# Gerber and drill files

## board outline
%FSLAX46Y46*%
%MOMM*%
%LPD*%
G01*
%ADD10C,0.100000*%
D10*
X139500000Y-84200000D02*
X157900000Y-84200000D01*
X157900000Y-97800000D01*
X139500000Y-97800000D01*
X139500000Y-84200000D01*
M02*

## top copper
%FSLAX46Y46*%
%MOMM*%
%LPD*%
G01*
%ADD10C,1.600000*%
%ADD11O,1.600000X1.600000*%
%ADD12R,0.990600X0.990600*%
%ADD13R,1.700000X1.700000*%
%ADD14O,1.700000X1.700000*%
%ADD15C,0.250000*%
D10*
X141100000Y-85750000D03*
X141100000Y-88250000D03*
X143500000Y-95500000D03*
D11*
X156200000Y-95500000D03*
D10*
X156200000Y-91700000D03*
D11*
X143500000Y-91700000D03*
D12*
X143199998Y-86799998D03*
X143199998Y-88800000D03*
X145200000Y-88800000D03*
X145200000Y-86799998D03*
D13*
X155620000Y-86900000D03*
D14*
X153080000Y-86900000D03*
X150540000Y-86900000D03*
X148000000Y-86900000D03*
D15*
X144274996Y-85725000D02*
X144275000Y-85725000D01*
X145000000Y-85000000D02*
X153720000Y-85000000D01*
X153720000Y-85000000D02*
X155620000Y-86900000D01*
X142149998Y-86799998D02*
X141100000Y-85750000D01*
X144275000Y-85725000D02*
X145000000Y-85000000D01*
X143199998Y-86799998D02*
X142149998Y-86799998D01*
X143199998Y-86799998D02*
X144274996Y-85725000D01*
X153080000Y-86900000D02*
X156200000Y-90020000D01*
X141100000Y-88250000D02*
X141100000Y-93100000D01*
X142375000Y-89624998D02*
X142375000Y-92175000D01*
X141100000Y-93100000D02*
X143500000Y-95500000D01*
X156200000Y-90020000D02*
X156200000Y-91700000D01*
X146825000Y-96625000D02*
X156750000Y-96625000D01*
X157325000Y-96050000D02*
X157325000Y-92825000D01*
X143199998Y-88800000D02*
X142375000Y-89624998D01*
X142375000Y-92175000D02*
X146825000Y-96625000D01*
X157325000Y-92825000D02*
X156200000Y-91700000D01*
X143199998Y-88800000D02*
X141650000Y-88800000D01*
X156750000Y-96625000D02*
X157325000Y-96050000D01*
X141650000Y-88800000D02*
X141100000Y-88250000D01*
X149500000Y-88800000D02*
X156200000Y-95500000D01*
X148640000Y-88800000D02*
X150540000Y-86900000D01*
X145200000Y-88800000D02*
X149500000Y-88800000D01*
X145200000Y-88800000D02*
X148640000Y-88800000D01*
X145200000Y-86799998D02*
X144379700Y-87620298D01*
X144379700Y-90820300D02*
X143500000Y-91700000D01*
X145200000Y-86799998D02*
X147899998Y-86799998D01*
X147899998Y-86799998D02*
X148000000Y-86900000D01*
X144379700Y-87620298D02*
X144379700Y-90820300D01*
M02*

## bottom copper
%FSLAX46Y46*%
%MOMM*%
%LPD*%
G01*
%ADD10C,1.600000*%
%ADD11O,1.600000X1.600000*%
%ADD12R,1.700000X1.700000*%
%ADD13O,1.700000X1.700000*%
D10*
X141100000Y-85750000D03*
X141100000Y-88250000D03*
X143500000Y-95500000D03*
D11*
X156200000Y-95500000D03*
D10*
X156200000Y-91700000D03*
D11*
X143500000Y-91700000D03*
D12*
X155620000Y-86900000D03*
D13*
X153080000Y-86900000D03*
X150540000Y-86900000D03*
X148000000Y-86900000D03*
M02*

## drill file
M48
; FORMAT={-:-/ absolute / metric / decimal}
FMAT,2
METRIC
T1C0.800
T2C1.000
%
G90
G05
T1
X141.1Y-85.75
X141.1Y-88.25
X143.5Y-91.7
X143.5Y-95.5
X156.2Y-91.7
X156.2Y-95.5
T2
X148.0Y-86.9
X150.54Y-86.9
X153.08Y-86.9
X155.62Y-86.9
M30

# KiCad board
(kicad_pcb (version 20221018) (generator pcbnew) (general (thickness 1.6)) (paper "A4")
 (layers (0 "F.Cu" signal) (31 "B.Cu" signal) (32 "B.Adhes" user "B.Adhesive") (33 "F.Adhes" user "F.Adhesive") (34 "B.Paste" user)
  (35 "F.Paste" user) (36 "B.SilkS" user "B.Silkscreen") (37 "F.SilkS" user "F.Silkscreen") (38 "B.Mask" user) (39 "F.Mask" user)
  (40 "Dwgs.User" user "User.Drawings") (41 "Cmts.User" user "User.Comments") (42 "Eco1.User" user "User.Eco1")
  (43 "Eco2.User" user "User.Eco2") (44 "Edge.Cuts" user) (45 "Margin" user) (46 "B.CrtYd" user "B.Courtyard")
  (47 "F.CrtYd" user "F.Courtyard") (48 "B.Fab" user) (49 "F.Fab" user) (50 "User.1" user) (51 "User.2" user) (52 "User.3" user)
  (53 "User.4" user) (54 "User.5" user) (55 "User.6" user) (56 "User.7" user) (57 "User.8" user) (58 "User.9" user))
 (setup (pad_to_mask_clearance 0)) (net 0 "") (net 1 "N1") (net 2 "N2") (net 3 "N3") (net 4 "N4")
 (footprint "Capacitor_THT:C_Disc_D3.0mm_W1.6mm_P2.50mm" (layer "F.Cu") (at 141.1 85.75 -90)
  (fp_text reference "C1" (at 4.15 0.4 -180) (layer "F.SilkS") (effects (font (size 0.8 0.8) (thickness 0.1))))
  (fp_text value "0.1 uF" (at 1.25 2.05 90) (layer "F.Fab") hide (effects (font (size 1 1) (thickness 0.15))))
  (pad "1" thru_hole circle (at 0 0 270) (size 1.6 1.6) (drill 0.8) (layers "*.Cu" "*.Mask") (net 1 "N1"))
  (pad "2" thru_hole circle (at 2.5 0 270) (size 1.6 1.6) (drill 0.8) (layers "*.Cu" "*.Mask") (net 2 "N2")))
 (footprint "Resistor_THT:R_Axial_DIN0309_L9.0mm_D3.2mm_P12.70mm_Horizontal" (layer "F.Cu") (at 143.5 95.5)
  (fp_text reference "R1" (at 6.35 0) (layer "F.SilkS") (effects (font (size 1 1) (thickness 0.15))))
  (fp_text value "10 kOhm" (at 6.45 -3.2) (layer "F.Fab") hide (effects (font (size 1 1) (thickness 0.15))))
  (pad "1" thru_hole circle (at 0 0) (size 1.6 1.6) (drill 0.8) (layers "*.Cu" "*.Mask") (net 2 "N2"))
  (pad "2" thru_hole oval (at 12.7 0) (size 1.6 1.6) (drill 0.8) (layers "*.Cu" "*.Mask") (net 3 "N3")))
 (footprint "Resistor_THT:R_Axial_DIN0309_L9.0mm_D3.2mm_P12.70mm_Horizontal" (layer "F.Cu") (at 156.2 91.7 180)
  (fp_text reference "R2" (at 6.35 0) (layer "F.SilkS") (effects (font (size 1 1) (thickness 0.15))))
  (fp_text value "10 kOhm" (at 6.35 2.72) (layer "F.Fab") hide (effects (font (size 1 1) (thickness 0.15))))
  (pad "1" thru_hole circle (at 0 0 180) (size 1.6 1.6) (drill 0.8) (layers "*.Cu" "*.Mask") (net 2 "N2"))
  (pad "2" thru_hole oval (at 12.7 0 180) (size 1.6 1.6) (drill 0.8) (layers "*.Cu" "*.Mask") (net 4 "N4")))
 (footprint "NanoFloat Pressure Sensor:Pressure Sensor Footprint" (layer "F.Cu") (at 144.199999 87.799999)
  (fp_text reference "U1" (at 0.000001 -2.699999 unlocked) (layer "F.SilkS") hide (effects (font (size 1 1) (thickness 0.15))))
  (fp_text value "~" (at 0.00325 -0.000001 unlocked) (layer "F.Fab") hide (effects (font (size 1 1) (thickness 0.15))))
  (pad "1" smd rect (at -1.000001 -1.000001) (size 0.9906 0.9906) (layers "F.Cu" "F.Paste" "F.Mask") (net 1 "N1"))
  (pad "2" smd rect (at -1.000001 1.000001) (size 0.9906 0.9906) (layers "F.Cu" "F.Paste" "F.Mask") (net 2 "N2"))
  (pad "3" smd rect (at 1.000001 1.000001) (size 0.9906 0.9906) (layers "F.Cu" "F.Paste" "F.Mask") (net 3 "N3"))
  (pad "4" smd rect (at 1.000001 -1.000001) (size 0.9906 0.9906) (layers "F.Cu" "F.Paste" "F.Mask") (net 4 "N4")))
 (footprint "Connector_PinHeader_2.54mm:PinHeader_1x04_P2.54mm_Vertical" (layer "B.Cu") (at 155.62 86.9 90)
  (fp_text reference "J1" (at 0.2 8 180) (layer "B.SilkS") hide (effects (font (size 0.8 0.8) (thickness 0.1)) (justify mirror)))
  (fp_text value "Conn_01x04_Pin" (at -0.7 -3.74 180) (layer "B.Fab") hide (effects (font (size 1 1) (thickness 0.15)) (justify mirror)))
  (pad "1" thru_hole rect (at 0 0 90) (size 1.7 1.7) (drill 1) (layers "*.Cu" "*.Mask") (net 1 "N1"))
  (pad "2" thru_hole oval (at 0 -2.54 90) (size 1.7 1.7) (drill 1) (layers "*.Cu" "*.Mask") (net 2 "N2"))
  (pad "3" thru_hole oval (at 0 -5.08 90) (size 1.7 1.7) (drill 1) (layers "*.Cu" "*.Mask") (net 3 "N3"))
  (pad "4" thru_hole oval (at 0 -7.62 90) (size 1.7 1.7) (drill 1) (layers "*.Cu" "*.Mask") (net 4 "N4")))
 (gr_rect (start 139.5 84.2) (end 157.9 97.8) (stroke (width 0.1) (type default)) (fill none) (layer "Edge.Cuts"))
 (segment (start 144.274996 85.725) (end 144.275 85.725) (width 0.25) (layer "F.Cu") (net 1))
 (segment (start 145 85) (end 153.72 85) (width 0.25) (layer "F.Cu") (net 1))
 (segment (start 153.72 85) (end 155.62 86.9) (width 0.25) (layer "F.Cu") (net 1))
 (segment (start 142.149998 86.799998) (end 141.1 85.75) (width 0.25) (layer "F.Cu") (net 1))
 (segment (start 144.275 85.725) (end 145 85) (width 0.25) (layer "F.Cu") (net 1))
 (segment (start 143.199998 86.799998) (end 142.149998 86.799998) (width 0.25) (layer "F.Cu") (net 1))
 (segment (start 143.199998 86.799998) (end 144.274996 85.725) (width 0.25) (layer "F.Cu") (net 1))
 (segment (start 153.08 86.9) (end 156.2 90.02) (width 0.25) (layer "F.Cu") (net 2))
 (segment (start 141.1 88.25) (end 141.1 93.1) (width 0.25) (layer "F.Cu") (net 2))
 (segment (start 142.375 89.624998) (end 142.375 92.175) (width 0.25) (layer "F.Cu") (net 2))
 (segment (start 141.1 93.1) (end 143.5 95.5) (width 0.25) (layer "F.Cu") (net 2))
 (segment (start 156.2 90.02) (end 156.2 91.7) (width 0.25) (layer "F.Cu") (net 2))
 (segment (start 146.825 96.625) (end 156.75 96.625) (width 0.25) (layer "F.Cu") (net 2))
 (segment (start 157.325 96.05) (end 157.325 92.825) (width 0.25) (layer "F.Cu") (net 2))
 (segment (start 143.199998 88.8) (end 142.375 89.624998) (width 0.25) (layer "F.Cu") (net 2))
 (segment (start 142.375 92.175) (end 146.825 96.625) (width 0.25) (layer "F.Cu") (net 2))
 (segment (start 157.325 92.825) (end 156.2 91.7) (width 0.25) (layer "F.Cu") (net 2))
 (segment (start 143.199998 88.8) (end 141.65 88.8) (width 0.25) (layer "F.Cu") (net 2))
 (segment (start 156.75 96.625) (end 157.325 96.05) (width 0.25) (layer "F.Cu") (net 2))
 (segment (start 141.65 88.8) (end 141.1 88.25) (width 0.25) (layer "F.Cu") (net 2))
 (segment (start 149.5 88.8) (end 156.2 95.5) (width 0.25) (layer "F.Cu") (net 3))
 (segment (start 148.64 88.8) (end 150.54 86.9) (width 0.25) (layer "F.Cu") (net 3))
 (segment (start 145.2 88.8) (end 149.5 88.8) (width 0.25) (layer "F.Cu") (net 3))
 (segment (start 145.2 88.8) (end 148.64 88.8) (width 0.25) (layer "F.Cu") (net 3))
 (segment (start 145.2 86.799998) (end 144.3797 87.620298) (width 0.25) (layer "F.Cu") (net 4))
 (segment (start 144.3797 90.8203) (end 143.5 91.7) (width 0.25) (layer "F.Cu") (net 4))
 (segment (start 145.2 86.799998) (end 147.899998 86.799998) (width 0.25) (layer "F.Cu") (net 4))
 (segment (start 147.899998 86.799998) (end 148 86.9) (width 0.25) (layer "F.Cu") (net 4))
 (segment (start 144.3797 87.620298) (end 144.3797 90.8203) (width 0.25) (layer "F.Cu") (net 4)))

